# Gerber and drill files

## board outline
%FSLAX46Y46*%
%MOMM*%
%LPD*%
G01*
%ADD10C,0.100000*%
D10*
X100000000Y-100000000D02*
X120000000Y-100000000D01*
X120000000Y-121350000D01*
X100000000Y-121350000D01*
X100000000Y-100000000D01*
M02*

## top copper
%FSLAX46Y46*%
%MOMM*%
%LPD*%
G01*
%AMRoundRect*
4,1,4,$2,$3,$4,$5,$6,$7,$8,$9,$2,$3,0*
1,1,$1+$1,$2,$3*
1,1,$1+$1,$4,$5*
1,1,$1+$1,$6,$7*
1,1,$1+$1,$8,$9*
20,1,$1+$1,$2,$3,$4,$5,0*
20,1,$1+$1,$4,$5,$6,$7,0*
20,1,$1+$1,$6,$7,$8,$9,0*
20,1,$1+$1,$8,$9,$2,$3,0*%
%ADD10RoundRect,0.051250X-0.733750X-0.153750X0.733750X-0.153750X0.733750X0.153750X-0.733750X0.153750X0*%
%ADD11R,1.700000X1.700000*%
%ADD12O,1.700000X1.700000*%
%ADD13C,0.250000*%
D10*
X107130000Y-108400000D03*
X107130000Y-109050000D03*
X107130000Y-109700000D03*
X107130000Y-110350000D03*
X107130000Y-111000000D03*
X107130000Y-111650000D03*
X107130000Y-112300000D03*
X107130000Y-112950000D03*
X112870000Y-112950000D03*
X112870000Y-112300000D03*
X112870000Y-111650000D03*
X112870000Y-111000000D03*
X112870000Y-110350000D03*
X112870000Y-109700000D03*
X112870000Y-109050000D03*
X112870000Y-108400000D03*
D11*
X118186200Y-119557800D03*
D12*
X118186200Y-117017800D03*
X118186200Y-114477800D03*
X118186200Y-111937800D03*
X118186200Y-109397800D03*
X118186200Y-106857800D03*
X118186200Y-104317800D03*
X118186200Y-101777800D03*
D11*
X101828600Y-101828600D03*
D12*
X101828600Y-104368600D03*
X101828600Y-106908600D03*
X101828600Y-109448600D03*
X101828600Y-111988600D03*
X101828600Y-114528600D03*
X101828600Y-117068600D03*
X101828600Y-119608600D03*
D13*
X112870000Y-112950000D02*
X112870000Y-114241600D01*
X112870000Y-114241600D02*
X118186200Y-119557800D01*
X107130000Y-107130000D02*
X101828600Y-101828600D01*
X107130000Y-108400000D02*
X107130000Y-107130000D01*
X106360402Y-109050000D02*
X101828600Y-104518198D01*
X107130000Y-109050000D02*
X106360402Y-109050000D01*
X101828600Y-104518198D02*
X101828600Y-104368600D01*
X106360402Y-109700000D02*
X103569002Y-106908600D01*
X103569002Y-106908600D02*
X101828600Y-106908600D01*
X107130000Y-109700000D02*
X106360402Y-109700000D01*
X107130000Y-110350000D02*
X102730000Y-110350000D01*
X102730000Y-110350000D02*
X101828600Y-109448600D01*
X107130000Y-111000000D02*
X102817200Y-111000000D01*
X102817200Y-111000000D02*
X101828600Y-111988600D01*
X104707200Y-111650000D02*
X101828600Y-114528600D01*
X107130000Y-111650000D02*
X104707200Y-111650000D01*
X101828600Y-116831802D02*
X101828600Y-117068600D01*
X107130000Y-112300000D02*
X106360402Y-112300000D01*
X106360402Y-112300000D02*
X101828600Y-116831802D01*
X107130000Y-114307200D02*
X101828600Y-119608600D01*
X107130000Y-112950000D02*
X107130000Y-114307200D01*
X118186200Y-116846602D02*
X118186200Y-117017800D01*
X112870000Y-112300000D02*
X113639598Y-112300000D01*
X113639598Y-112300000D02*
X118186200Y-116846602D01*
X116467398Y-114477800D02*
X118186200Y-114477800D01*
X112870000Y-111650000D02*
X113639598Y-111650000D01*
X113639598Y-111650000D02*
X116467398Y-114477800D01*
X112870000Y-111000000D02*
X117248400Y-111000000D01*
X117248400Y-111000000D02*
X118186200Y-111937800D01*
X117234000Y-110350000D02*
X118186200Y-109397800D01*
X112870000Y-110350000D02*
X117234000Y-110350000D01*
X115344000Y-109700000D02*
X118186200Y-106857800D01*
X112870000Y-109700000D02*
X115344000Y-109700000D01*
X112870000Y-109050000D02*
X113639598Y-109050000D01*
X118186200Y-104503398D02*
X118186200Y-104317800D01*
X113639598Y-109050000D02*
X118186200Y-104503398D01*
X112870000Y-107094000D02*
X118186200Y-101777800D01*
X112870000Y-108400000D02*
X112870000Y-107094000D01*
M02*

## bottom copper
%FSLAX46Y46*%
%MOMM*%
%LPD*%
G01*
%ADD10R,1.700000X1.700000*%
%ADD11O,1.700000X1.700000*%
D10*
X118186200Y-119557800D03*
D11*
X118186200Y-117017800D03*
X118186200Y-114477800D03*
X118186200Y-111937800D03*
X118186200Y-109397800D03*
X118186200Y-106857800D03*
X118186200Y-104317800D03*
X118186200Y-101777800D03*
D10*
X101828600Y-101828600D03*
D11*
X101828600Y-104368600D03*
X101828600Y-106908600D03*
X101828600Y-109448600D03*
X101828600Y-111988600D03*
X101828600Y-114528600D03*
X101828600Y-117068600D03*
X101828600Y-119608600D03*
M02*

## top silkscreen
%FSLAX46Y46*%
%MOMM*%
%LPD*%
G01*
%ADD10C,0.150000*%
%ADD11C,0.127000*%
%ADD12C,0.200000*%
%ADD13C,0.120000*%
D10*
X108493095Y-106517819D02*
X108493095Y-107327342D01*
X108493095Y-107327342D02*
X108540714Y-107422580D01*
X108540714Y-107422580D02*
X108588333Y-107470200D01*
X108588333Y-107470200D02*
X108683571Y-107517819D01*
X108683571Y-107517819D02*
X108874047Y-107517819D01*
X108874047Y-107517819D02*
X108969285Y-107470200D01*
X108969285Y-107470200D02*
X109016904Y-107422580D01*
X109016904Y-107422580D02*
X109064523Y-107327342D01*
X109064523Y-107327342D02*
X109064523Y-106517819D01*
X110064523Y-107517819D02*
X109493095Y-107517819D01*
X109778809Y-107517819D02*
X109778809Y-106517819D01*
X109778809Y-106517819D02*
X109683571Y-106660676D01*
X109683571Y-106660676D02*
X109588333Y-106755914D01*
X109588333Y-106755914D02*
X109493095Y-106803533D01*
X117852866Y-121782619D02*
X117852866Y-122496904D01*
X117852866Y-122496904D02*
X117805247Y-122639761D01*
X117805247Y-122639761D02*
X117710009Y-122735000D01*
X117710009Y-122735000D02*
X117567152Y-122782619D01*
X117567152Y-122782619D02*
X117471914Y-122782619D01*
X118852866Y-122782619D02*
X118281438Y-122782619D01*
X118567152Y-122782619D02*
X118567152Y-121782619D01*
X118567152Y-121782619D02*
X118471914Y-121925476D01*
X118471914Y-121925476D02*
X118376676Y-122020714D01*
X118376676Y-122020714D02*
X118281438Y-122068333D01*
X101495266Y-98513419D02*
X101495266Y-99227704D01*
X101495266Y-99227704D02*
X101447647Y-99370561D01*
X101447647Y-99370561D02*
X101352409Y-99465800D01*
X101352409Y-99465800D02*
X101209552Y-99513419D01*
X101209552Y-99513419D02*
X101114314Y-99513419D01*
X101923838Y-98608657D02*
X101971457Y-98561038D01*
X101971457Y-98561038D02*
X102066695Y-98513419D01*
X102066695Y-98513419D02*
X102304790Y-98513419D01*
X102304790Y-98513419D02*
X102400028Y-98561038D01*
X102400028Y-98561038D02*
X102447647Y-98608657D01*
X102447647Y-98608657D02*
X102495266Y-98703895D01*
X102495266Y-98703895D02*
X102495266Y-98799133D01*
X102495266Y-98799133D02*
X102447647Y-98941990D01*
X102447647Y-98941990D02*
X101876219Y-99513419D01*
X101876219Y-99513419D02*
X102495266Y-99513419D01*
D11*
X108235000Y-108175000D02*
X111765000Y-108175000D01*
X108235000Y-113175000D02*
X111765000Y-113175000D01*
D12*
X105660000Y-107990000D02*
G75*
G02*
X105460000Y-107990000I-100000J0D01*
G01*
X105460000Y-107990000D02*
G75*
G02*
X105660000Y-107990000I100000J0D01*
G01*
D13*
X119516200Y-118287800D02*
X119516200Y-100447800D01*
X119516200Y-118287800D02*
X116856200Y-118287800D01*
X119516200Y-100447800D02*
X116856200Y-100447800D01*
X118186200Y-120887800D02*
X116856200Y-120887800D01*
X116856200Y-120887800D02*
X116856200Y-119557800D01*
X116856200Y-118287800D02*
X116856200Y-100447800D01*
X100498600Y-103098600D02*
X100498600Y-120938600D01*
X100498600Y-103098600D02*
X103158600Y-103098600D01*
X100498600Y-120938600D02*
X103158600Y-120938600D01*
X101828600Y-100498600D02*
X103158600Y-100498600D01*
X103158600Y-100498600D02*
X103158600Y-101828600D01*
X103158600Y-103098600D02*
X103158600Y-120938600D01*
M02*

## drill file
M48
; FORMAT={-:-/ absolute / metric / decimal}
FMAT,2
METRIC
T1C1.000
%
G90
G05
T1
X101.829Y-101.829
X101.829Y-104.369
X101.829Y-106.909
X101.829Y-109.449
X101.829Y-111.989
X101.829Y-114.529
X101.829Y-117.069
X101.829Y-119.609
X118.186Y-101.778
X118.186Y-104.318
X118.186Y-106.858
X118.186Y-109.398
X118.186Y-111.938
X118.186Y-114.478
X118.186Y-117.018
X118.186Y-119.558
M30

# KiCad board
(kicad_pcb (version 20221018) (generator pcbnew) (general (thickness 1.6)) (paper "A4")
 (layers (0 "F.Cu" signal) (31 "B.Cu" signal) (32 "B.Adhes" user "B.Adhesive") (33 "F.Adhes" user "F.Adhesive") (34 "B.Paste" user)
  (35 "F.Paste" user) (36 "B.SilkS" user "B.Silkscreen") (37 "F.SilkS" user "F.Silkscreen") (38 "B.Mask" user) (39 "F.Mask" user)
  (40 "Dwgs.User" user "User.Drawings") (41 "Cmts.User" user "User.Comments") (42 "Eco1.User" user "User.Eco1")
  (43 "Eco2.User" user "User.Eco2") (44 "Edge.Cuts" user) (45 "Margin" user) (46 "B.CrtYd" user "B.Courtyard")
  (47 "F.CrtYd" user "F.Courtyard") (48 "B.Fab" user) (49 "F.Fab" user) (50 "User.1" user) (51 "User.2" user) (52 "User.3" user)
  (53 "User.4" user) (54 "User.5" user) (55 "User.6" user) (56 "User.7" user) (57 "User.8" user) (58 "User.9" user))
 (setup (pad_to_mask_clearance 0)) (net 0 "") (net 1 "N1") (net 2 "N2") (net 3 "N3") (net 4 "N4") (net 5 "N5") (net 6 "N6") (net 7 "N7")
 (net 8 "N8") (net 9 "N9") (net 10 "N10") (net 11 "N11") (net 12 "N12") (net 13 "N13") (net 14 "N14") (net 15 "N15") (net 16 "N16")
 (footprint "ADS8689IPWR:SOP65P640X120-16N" (layer "F.Cu") (at 110 110.675)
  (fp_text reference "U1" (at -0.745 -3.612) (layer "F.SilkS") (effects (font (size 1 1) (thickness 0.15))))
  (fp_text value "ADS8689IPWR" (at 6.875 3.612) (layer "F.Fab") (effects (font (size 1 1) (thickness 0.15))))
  (fp_line (start -1.765 -2.5) (end 1.765 -2.5) (stroke (width 0.127) (type solid)) (layer "F.SilkS"))
  (fp_line (start -1.765 2.5) (end 1.765 2.5) (stroke (width 0.127) (type solid)) (layer "F.SilkS"))
  (fp_circle (center -4.44 -2.685) (end -4.34 -2.685) (stroke (width 0.2) (type solid)) (fill none) (layer "F.SilkS"))
  (pad "1" smd roundrect (at -2.87 -2.275) (size 1.57 0.41) (layers "F.Cu" "F.Paste" "F.Mask") (roundrect_rratio 0.125) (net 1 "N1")
   (solder_mask_margin 0.102))
  (pad "2" smd roundrect (at -2.87 -1.625) (size 1.57 0.41) (layers "F.Cu" "F.Paste" "F.Mask") (roundrect_rratio 0.125) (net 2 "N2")
   (solder_mask_margin 0.102))
  (pad "3" smd roundrect (at -2.87 -0.975) (size 1.57 0.41) (layers "F.Cu" "F.Paste" "F.Mask") (roundrect_rratio 0.125) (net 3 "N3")
   (solder_mask_margin 0.102))
  (pad "4" smd roundrect (at -2.87 -0.325) (size 1.57 0.41) (layers "F.Cu" "F.Paste" "F.Mask") (roundrect_rratio 0.125) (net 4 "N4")
   (solder_mask_margin 0.102))
  (pad "5" smd roundrect (at -2.87 0.325) (size 1.57 0.41) (layers "F.Cu" "F.Paste" "F.Mask") (roundrect_rratio 0.125) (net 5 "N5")
   (solder_mask_margin 0.102))
  (pad "6" smd roundrect (at -2.87 0.975) (size 1.57 0.41) (layers "F.Cu" "F.Paste" "F.Mask") (roundrect_rratio 0.125) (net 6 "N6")
   (solder_mask_margin 0.102))
  (pad "7" smd roundrect (at -2.87 1.625) (size 1.57 0.41) (layers "F.Cu" "F.Paste" "F.Mask") (roundrect_rratio 0.125) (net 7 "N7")
   (solder_mask_margin 0.102))
  (pad "8" smd roundrect (at -2.87 2.275) (size 1.57 0.41) (layers "F.Cu" "F.Paste" "F.Mask") (roundrect_rratio 0.125) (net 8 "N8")
   (solder_mask_margin 0.102))
  (pad "9" smd roundrect (at 2.87 2.275) (size 1.57 0.41) (layers "F.Cu" "F.Paste" "F.Mask") (roundrect_rratio 0.125) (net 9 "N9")
   (solder_mask_margin 0.102))
  (pad "10" smd roundrect (at 2.87 1.625) (size 1.57 0.41) (layers "F.Cu" "F.Paste" "F.Mask") (roundrect_rratio 0.125) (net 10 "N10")
   (solder_mask_margin 0.102))
  (pad "11" smd roundrect (at 2.87 0.975) (size 1.57 0.41) (layers "F.Cu" "F.Paste" "F.Mask") (roundrect_rratio 0.125) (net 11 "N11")
   (solder_mask_margin 0.102))
  (pad "12" smd roundrect (at 2.87 0.325) (size 1.57 0.41) (layers "F.Cu" "F.Paste" "F.Mask") (roundrect_rratio 0.125) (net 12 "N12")
   (solder_mask_margin 0.102))
  (pad "13" smd roundrect (at 2.87 -0.325) (size 1.57 0.41) (layers "F.Cu" "F.Paste" "F.Mask") (roundrect_rratio 0.125) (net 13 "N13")
   (solder_mask_margin 0.102))
  (pad "14" smd roundrect (at 2.87 -0.975) (size 1.57 0.41) (layers "F.Cu" "F.Paste" "F.Mask") (roundrect_rratio 0.125) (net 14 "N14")
   (solder_mask_margin 0.102))
  (pad "15" smd roundrect (at 2.87 -1.625) (size 1.57 0.41) (layers "F.Cu" "F.Paste" "F.Mask") (roundrect_rratio 0.125) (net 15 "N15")
   (solder_mask_margin 0.102))
  (pad "16" smd roundrect (at 2.87 -2.275) (size 1.57 0.41) (layers "F.Cu" "F.Paste" "F.Mask") (roundrect_rratio 0.125) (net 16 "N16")
   (solder_mask_margin 0.102)))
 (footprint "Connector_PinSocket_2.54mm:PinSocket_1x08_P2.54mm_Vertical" (layer "F.Cu") (at 118.1862 119.5578 180)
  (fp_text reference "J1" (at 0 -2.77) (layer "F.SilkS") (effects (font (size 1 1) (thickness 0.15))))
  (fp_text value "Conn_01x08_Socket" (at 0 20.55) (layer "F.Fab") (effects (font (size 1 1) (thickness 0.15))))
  (fp_line (start -1.33 1.27) (end -1.33 19.11) (stroke (width 0.12) (type solid)) (layer "F.SilkS"))
  (fp_line (start -1.33 1.27) (end 1.33 1.27) (stroke (width 0.12) (type solid)) (layer "F.SilkS"))
  (fp_line (start -1.33 19.11) (end 1.33 19.11) (stroke (width 0.12) (type solid)) (layer "F.SilkS"))
  (fp_line (start 0 -1.33) (end 1.33 -1.33) (stroke (width 0.12) (type solid)) (layer "F.SilkS"))
  (fp_line (start 1.33 -1.33) (end 1.33 0) (stroke (width 0.12) (type solid)) (layer "F.SilkS"))
  (fp_line (start 1.33 1.27) (end 1.33 19.11) (stroke (width 0.12) (type solid)) (layer "F.SilkS"))
  (pad "1" thru_hole rect (at 0 0 180) (size 1.7 1.7) (drill 1) (layers "*.Cu" "*.Mask") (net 9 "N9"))
  (pad "2" thru_hole oval (at 0 2.54 180) (size 1.7 1.7) (drill 1) (layers "*.Cu" "*.Mask") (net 10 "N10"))
  (pad "3" thru_hole oval (at 0 5.08 180) (size 1.7 1.7) (drill 1) (layers "*.Cu" "*.Mask") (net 11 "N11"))
  (pad "4" thru_hole oval (at 0 7.62 180) (size 1.7 1.7) (drill 1) (layers "*.Cu" "*.Mask") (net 12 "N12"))
  (pad "5" thru_hole oval (at 0 10.16 180) (size 1.7 1.7) (drill 1) (layers "*.Cu" "*.Mask") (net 13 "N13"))
  (pad "6" thru_hole oval (at 0 12.7 180) (size 1.7 1.7) (drill 1) (layers "*.Cu" "*.Mask") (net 14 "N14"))
  (pad "7" thru_hole oval (at 0 15.24 180) (size 1.7 1.7) (drill 1) (layers "*.Cu" "*.Mask") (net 15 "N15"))
  (pad "8" thru_hole oval (at 0 17.78 180) (size 1.7 1.7) (drill 1) (layers "*.Cu" "*.Mask") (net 16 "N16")))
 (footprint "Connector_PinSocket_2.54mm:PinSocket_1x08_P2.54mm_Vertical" (layer "F.Cu") (at 101.8286 101.8286)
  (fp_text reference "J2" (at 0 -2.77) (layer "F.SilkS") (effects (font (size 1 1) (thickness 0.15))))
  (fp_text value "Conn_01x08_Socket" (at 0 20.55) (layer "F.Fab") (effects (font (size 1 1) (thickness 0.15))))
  (fp_line (start -1.33 1.27) (end -1.33 19.11) (stroke (width 0.12) (type solid)) (layer "F.SilkS"))
  (fp_line (start -1.33 1.27) (end 1.33 1.27) (stroke (width 0.12) (type solid)) (layer "F.SilkS"))
  (fp_line (start -1.33 19.11) (end 1.33 19.11) (stroke (width 0.12) (type solid)) (layer "F.SilkS"))
  (fp_line (start 0 -1.33) (end 1.33 -1.33) (stroke (width 0.12) (type solid)) (layer "F.SilkS"))
  (fp_line (start 1.33 -1.33) (end 1.33 0) (stroke (width 0.12) (type solid)) (layer "F.SilkS"))
  (fp_line (start 1.33 1.27) (end 1.33 19.11) (stroke (width 0.12) (type solid)) (layer "F.SilkS"))
  (pad "1" thru_hole rect (at 0 0) (size 1.7 1.7) (drill 1) (layers "*.Cu" "*.Mask") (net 1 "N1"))
  (pad "2" thru_hole oval (at 0 2.54) (size 1.7 1.7) (drill 1) (layers "*.Cu" "*.Mask") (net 2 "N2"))
  (pad "3" thru_hole oval (at 0 5.08) (size 1.7 1.7) (drill 1) (layers "*.Cu" "*.Mask") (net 3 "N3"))
  (pad "4" thru_hole oval (at 0 7.62) (size 1.7 1.7) (drill 1) (layers "*.Cu" "*.Mask") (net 4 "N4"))
  (pad "5" thru_hole oval (at 0 10.16) (size 1.7 1.7) (drill 1) (layers "*.Cu" "*.Mask") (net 5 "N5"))
  (pad "6" thru_hole oval (at 0 12.7) (size 1.7 1.7) (drill 1) (layers "*.Cu" "*.Mask") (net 6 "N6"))
  (pad "7" thru_hole oval (at 0 15.24) (size 1.7 1.7) (drill 1) (layers "*.Cu" "*.Mask") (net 7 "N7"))
  (pad "8" thru_hole oval (at 0 17.78) (size 1.7 1.7) (drill 1) (layers "*.Cu" "*.Mask") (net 8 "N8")))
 (gr_rect (start 100 100) (end 120 121.35) (stroke (width 0.1) (type default)) (fill none) (layer "Edge.Cuts"))
 (segment (start 112.87 112.95) (end 112.87 114.2416) (width 0.25) (layer "F.Cu") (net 9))
 (segment (start 112.87 114.2416) (end 118.1862 119.5578) (width 0.25) (layer "F.Cu") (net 9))
 (segment (start 107.13 107.13) (end 101.8286 101.8286) (width 0.25) (layer "F.Cu") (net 1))
 (segment (start 107.13 108.4) (end 107.13 107.13) (width 0.25) (layer "F.Cu") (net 1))
 (segment (start 106.360402 109.05) (end 101.8286 104.518198) (width 0.25) (layer "F.Cu") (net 2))
 (segment (start 107.13 109.05) (end 106.360402 109.05) (width 0.25) (layer "F.Cu") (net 2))
 (segment (start 101.8286 104.518198) (end 101.8286 104.3686) (width 0.25) (layer "F.Cu") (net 2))
 (segment (start 106.360402 109.7) (end 103.569002 106.9086) (width 0.25) (layer "F.Cu") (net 3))
 (segment (start 103.569002 106.9086) (end 101.8286 106.9086) (width 0.25) (layer "F.Cu") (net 3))
 (segment (start 107.13 109.7) (end 106.360402 109.7) (width 0.25) (layer "F.Cu") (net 3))
 (segment (start 107.13 110.35) (end 102.73 110.35) (width 0.25) (layer "F.Cu") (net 4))
 (segment (start 102.73 110.35) (end 101.8286 109.4486) (width 0.25) (layer "F.Cu") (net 4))
 (segment (start 107.13 111) (end 102.8172 111) (width 0.25) (layer "F.Cu") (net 5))
 (segment (start 102.8172 111) (end 101.8286 111.9886) (width 0.25) (layer "F.Cu") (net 5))
 (segment (start 104.7072 111.65) (end 101.8286 114.5286) (width 0.25) (layer "F.Cu") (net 6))
 (segment (start 107.13 111.65) (end 104.7072 111.65) (width 0.25) (layer "F.Cu") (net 6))
 (segment (start 101.8286 116.831802) (end 101.8286 117.0686) (width 0.25) (layer "F.Cu") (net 7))
 (segment (start 107.13 112.3) (end 106.360402 112.3) (width 0.25) (layer "F.Cu") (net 7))
 (segment (start 106.360402 112.3) (end 101.8286 116.831802) (width 0.25) (layer "F.Cu") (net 7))
 (segment (start 107.13 114.3072) (end 101.8286 119.6086) (width 0.25) (layer "F.Cu") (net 8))
 (segment (start 107.13 112.95) (end 107.13 114.3072) (width 0.25) (layer "F.Cu") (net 8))
 (segment (start 118.1862 116.846602) (end 118.1862 117.0178) (width 0.25) (layer "F.Cu") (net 10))
 (segment (start 112.87 112.3) (end 113.639598 112.3) (width 0.25) (layer "F.Cu") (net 10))
 (segment (start 113.639598 112.3) (end 118.1862 116.846602) (width 0.25) (layer "F.Cu") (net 10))
 (segment (start 116.467398 114.4778) (end 118.1862 114.4778) (width 0.25) (layer "F.Cu") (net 11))
 (segment (start 112.87 111.65) (end 113.639598 111.65) (width 0.25) (layer "F.Cu") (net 11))
 (segment (start 113.639598 111.65) (end 116.467398 114.4778) (width 0.25) (layer "F.Cu") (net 11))
 (segment (start 112.87 111) (end 117.2484 111) (width 0.25) (layer "F.Cu") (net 12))
 (segment (start 117.2484 111) (end 118.1862 111.9378) (width 0.25) (layer "F.Cu") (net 12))
 (segment (start 117.234 110.35) (end 118.1862 109.3978) (width 0.25) (layer "F.Cu") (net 13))
 (segment (start 112.87 110.35) (end 117.234 110.35) (width 0.25) (layer "F.Cu") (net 13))
 (segment (start 115.344 109.7) (end 118.1862 106.8578) (width 0.25) (layer "F.Cu") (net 14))
 (segment (start 112.87 109.7) (end 115.344 109.7) (width 0.25) (layer "F.Cu") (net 14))
 (segment (start 112.87 109.05) (end 113.639598 109.05) (width 0.25) (layer "F.Cu") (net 15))
 (segment (start 118.1862 104.503398) (end 118.1862 104.3178) (width 0.25) (layer "F.Cu") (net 15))
 (segment (start 113.639598 109.05) (end 118.1862 104.503398) (width 0.25) (layer "F.Cu") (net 15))
 (segment (start 112.87 107.094) (end 118.1862 101.7778) (width 0.25) (layer "F.Cu") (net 16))
 (segment (start 112.87 108.4) (end 112.87 107.094) (width 0.25) (layer "F.Cu") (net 16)))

